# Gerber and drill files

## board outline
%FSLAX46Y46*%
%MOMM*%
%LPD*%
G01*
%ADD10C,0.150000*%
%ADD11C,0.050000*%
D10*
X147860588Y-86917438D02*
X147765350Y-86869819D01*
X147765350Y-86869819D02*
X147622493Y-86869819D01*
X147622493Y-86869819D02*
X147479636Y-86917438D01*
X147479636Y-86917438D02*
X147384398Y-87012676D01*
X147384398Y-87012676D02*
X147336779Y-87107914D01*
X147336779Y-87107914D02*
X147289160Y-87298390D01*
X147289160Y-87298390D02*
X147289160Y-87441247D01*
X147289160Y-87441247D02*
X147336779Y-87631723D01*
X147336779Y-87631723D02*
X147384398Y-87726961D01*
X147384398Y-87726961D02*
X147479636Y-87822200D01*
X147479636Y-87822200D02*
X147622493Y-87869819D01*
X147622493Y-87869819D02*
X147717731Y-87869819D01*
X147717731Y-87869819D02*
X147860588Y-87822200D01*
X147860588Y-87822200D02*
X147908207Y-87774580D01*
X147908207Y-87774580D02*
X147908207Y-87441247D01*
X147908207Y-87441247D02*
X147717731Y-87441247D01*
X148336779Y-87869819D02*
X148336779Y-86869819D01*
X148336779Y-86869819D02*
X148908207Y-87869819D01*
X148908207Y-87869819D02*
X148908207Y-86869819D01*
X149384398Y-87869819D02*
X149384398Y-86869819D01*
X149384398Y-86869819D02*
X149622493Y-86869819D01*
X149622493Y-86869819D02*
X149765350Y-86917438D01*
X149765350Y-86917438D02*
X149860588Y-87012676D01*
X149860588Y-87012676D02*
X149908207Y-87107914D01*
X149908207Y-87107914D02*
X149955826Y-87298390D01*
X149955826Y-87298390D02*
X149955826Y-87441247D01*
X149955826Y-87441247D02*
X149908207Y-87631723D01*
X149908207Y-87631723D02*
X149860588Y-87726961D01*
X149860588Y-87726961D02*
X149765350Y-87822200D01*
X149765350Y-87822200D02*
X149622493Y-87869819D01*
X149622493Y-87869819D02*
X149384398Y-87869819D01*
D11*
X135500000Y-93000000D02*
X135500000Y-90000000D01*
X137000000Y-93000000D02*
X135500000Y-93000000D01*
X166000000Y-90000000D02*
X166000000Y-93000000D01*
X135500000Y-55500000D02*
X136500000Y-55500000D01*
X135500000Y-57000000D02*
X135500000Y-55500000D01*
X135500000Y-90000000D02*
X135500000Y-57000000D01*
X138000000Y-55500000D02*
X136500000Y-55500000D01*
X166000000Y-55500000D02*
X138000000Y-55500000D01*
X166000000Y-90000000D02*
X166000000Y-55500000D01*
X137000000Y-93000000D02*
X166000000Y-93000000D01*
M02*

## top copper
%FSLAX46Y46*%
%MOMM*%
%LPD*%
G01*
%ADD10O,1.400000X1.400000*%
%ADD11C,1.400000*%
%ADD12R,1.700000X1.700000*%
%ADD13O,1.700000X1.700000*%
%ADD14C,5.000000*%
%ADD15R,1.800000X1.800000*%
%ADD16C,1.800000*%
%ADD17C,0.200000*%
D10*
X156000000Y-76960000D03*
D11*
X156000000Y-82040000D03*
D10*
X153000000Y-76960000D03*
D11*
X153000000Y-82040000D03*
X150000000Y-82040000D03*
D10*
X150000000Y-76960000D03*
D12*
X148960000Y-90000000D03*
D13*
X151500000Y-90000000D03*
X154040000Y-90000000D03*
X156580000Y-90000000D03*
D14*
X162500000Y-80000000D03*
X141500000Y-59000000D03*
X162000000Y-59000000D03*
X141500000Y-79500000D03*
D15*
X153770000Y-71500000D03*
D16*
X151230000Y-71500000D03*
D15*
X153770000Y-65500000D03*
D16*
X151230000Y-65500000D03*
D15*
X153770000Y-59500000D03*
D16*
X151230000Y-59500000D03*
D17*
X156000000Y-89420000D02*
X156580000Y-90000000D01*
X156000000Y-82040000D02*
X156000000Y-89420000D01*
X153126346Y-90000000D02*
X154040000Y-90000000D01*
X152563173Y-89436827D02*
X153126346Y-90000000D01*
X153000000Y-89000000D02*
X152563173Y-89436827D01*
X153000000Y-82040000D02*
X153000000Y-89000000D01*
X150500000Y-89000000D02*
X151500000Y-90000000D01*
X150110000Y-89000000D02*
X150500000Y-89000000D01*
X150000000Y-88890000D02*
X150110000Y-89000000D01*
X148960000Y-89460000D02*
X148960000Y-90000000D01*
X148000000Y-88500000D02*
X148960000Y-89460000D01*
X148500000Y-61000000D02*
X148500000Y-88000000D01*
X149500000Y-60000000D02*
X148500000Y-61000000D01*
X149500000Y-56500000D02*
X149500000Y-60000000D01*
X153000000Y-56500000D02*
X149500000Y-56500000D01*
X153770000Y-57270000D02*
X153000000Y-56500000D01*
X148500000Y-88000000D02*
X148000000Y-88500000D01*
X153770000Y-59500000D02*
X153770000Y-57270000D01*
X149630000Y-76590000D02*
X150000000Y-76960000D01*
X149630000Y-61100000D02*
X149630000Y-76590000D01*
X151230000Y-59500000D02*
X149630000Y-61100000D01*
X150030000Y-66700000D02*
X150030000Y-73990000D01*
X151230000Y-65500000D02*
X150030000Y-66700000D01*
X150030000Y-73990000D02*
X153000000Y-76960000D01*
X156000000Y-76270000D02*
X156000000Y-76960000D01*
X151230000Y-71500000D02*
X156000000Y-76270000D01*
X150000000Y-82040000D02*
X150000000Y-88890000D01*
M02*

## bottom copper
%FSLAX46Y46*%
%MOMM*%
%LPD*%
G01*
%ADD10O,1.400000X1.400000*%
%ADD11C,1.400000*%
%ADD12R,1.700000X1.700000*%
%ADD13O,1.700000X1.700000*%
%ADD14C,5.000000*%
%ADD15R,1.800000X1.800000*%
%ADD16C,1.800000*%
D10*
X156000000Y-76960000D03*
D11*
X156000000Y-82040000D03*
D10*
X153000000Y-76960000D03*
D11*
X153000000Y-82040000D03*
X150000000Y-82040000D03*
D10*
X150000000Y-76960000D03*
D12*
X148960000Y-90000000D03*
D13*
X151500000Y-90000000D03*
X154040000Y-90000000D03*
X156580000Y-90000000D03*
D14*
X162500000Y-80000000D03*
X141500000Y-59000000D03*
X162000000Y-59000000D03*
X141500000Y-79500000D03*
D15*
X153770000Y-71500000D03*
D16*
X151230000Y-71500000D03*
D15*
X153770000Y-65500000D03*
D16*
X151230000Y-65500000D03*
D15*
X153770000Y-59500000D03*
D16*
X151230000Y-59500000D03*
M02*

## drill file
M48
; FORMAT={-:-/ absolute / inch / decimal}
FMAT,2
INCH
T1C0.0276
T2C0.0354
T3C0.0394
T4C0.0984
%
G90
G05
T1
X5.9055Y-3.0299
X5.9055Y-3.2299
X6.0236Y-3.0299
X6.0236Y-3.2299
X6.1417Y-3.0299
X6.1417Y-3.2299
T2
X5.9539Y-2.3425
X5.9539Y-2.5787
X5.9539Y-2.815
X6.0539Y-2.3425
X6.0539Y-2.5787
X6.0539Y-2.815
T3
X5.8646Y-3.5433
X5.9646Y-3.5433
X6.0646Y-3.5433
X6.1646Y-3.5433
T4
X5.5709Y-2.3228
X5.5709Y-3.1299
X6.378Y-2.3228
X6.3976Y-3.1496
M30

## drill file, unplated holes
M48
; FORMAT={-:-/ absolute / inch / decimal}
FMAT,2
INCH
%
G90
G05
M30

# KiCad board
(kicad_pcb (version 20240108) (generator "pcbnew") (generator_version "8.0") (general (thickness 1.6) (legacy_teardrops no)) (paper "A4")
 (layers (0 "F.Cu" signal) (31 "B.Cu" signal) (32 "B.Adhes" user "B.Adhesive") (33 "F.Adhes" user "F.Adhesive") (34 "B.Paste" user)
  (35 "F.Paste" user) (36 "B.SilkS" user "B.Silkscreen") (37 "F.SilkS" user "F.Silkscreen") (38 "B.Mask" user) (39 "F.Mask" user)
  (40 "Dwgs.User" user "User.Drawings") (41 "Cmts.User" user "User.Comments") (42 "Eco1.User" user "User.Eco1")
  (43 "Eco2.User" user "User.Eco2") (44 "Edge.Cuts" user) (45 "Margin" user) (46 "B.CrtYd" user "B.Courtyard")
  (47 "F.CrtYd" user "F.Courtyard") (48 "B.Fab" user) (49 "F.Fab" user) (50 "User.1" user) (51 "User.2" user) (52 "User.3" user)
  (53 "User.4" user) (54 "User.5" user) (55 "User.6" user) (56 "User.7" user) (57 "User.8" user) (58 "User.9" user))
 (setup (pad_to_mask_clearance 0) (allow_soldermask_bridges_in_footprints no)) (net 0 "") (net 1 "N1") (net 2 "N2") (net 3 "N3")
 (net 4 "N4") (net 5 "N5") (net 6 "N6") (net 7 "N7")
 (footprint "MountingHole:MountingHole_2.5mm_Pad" (layer "F.Cu") (at 141.5 79.5)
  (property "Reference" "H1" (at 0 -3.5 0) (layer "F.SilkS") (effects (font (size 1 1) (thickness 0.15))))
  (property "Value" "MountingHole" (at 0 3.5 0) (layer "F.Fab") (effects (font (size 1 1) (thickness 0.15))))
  (pad "1" thru_hole circle (at 0 0) (size 5 5) (drill 2.5) (layers "*.Cu" "*.Mask") (remove_unused_layers no)))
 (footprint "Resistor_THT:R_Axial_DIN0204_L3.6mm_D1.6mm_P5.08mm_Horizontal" (layer "F.Cu") (at 156 82.04 90)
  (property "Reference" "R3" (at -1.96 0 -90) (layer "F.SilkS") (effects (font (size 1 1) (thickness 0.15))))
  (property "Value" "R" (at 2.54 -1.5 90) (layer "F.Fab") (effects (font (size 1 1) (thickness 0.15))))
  (pad "1" thru_hole circle (at 0 0 90) (size 1.4 1.4) (drill 0.7) (layers "*.Cu" "*.Mask") (remove_unused_layers no) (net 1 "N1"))
  (pad "2" thru_hole oval (at 5.08 0 90) (size 1.4 1.4) (drill 0.7) (layers "*.Cu" "*.Mask") (remove_unused_layers no) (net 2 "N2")))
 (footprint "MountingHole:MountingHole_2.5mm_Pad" (layer "F.Cu") (at 162.5 80)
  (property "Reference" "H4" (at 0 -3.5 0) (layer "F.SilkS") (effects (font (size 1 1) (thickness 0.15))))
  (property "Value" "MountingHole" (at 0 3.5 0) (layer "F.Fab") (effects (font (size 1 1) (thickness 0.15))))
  (pad "1" thru_hole circle (at 0 0) (size 5 5) (drill 2.5) (layers "*.Cu" "*.Mask") (remove_unused_layers no)))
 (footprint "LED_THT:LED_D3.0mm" (layer "F.Cu") (at 153.77 59.5 180)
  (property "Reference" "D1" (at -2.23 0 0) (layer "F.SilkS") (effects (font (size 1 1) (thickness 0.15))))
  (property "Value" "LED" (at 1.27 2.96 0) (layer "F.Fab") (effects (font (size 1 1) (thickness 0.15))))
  (pad "1" thru_hole rect (at 0 0 180) (size 1.8 1.8) (drill 0.9) (layers "*.Cu" "*.Mask") (remove_unused_layers no) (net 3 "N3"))
  (pad "2" thru_hole circle (at 2.54 0 180) (size 1.8 1.8) (drill 0.9) (layers "*.Cu" "*.Mask") (remove_unused_layers no) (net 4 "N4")))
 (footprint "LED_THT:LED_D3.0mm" (layer "F.Cu") (at 153.77 71.5 180)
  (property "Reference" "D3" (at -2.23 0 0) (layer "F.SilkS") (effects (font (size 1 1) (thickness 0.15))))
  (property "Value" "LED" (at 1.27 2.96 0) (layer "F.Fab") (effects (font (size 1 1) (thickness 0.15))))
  (pad "1" thru_hole rect (at 0 0 180) (size 1.8 1.8) (drill 0.9) (layers "*.Cu" "*.Mask") (remove_unused_layers no) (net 3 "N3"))
  (pad "2" thru_hole circle (at 2.54 0 180) (size 1.8 1.8) (drill 0.9) (layers "*.Cu" "*.Mask") (remove_unused_layers no) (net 2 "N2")))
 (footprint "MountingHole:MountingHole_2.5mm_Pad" (layer "F.Cu") (at 162 59)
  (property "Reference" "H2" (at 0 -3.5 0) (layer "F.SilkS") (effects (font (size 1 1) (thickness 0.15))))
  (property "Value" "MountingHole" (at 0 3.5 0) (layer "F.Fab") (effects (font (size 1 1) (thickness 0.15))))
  (pad "1" thru_hole circle (at 0 0) (size 5 5) (drill 2.5) (layers "*.Cu" "*.Mask") (remove_unused_layers no)))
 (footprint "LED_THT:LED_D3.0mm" (layer "F.Cu") (at 153.77 65.5 180)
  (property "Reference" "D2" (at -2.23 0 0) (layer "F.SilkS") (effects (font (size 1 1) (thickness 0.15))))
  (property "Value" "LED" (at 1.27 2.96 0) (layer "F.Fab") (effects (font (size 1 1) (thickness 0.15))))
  (pad "1" thru_hole rect (at 0 0 180) (size 1.8 1.8) (drill 0.9) (layers "*.Cu" "*.Mask") (remove_unused_layers no) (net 3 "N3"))
  (pad "2" thru_hole circle (at 2.54 0 180) (size 1.8 1.8) (drill 0.9) (layers "*.Cu" "*.Mask") (remove_unused_layers no) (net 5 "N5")))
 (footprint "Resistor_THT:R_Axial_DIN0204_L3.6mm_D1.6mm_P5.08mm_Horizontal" (layer "F.Cu") (at 153 82.04 90)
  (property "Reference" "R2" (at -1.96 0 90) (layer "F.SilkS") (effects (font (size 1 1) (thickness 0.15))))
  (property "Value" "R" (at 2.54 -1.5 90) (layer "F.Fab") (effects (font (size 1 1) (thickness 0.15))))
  (pad "1" thru_hole circle (at 0 0 90) (size 1.4 1.4) (drill 0.7) (layers "*.Cu" "*.Mask") (remove_unused_layers no) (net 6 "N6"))
  (pad "2" thru_hole oval (at 5.08 0 90) (size 1.4 1.4) (drill 0.7) (layers "*.Cu" "*.Mask") (remove_unused_layers no) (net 5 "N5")))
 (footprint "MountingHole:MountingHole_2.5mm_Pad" (layer "F.Cu") (at 141.5 59)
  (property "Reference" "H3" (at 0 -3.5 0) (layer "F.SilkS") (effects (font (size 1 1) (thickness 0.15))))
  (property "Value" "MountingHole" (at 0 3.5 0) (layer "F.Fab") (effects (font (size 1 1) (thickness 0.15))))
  (pad "1" thru_hole circle (at 0 0) (size 5 5) (drill 2.5) (layers "*.Cu" "*.Mask") (remove_unused_layers no)))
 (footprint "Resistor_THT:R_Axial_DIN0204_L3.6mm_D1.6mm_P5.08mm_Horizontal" (layer "F.Cu") (at 150 82.04 90)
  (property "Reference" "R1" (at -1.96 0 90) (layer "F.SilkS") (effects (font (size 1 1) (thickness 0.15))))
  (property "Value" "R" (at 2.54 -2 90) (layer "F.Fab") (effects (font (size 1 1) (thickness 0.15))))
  (pad "1" thru_hole circle (at 0 0 90) (size 1.4 1.4) (drill 0.7) (layers "*.Cu" "*.Mask") (remove_unused_layers no) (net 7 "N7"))
  (pad "2" thru_hole oval (at 5.08 0 90) (size 1.4 1.4) (drill 0.7) (layers "*.Cu" "*.Mask") (remove_unused_layers no) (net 4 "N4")))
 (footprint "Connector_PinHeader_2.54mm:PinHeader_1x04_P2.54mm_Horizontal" (layer "B.Cu") (at 148.96 90 -90)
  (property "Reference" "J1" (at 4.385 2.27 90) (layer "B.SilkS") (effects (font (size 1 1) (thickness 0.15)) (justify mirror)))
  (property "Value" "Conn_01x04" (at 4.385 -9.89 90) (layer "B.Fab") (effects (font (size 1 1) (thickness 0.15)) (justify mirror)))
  (pad "1" thru_hole rect (at 0 0 270) (size 1.7 1.7) (drill 1) (layers "*.Cu" "*.Mask") (remove_unused_layers no) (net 3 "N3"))
  (pad "2" thru_hole oval (at 0 -2.54 270) (size 1.7 1.7) (drill 1) (layers "*.Cu" "*.Mask") (remove_unused_layers no) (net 7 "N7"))
  (pad "3" thru_hole oval (at 0 -5.08 270) (size 1.7 1.7) (drill 1) (layers "*.Cu" "*.Mask") (remove_unused_layers no) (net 6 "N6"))
  (pad "4" thru_hole oval (at 0 -7.62 270) (size 1.7 1.7) (drill 1) (layers "*.Cu" "*.Mask") (remove_unused_layers no) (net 1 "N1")))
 (gr_line (start 166 55.5) (end 138 55.5) (stroke (width 0.05) (type default)) (layer "Edge.Cuts"))
 (gr_line (start 135.5 57) (end 135.5 55.5) (stroke (width 0.05) (type default)) (layer "Edge.Cuts"))
 (gr_line (start 137 93) (end 135.5 93) (stroke (width 0.05) (type default)) (layer "Edge.Cuts"))
 (gr_line (start 137 93) (end 166 93) (stroke (width 0.05) (type default)) (layer "Edge.Cuts"))
 (gr_line (start 138 55.5) (end 136.5 55.5) (stroke (width 0.05) (type default)) (layer "Edge.Cuts"))
 (gr_line (start 166 90) (end 166 93) (stroke (width 0.05) (type default)) (layer "Edge.Cuts"))
 (gr_line (start 135.5 93) (end 135.5 90) (stroke (width 0.05) (type default)) (layer "Edge.Cuts"))
 (gr_line (start 135.5 55.5) (end 136.5 55.5) (stroke (width 0.05) (type default)) (layer "Edge.Cuts"))
 (gr_line (start 166 90) (end 166 55.5) (stroke (width 0.05) (type default)) (layer "Edge.Cuts"))
 (gr_line (start 135.5 90) (end 135.5 57) (stroke (width 0.05) (type default)) (layer "Edge.Cuts"))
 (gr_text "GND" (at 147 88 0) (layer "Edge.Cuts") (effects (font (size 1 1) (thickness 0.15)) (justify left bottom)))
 (segment (start 149.5 56.5) (end 149.5 60) (width 0.2) (layer "F.Cu") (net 3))
 (segment (start 148.96 89.46) (end 148.96 90) (width 0.2) (layer "F.Cu") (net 3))
 (segment (start 153.77 59.5) (end 153.77 57.27) (width 0.2) (layer "F.Cu") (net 3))
 (segment (start 148.5 88) (end 148 88.5) (width 0.2) (layer "F.Cu") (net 3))
 (segment (start 149.5 60) (end 148.5 61) (width 0.2) (layer "F.Cu") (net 3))
 (segment (start 153 56.5) (end 149.5 56.5) (width 0.2) (layer "F.Cu") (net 3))
 (segment (start 148 88.5) (end 148.96 89.46) (width 0.2) (layer "F.Cu") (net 3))
 (segment (start 148.5 61) (end 148.5 88) (width 0.2) (layer "F.Cu") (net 3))
 (segment (start 153.77 57.27) (end 153 56.5) (width 0.2) (layer "F.Cu") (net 3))
 (segment (start 149.63 76.59) (end 150 76.96) (width 0.2) (layer "F.Cu") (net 4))
 (segment (start 149.63 61.1) (end 149.63 76.59) (width 0.2) (layer "F.Cu") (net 4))
 (segment (start 151.23 59.5) (end 149.63 61.1) (width 0.2) (layer "F.Cu") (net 4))
 (segment (start 150.03 66.7) (end 150.03 73.99) (width 0.2) (layer "F.Cu") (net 5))
 (segment (start 150.03 73.99) (end 153 76.96) (width 0.2) (layer "F.Cu") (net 5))
 (segment (start 151.23 65.5) (end 150.03 66.7) (width 0.2) (layer "F.Cu") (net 5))
 (segment (start 156 76.27) (end 156 76.96) (width 0.2) (layer "F.Cu") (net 2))
 (segment (start 151.23 71.5) (end 156 76.27) (width 0.2) (layer "F.Cu") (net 2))
 (segment (start 153 82.04) (end 153 89) (width 0.2) (layer "F.Cu") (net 6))
 (segment (start 152.563173 89.436827) (end 153.126346 90) (width 0.2) (layer "F.Cu") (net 6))
 (segment (start 153.126346 90) (end 154.04 90) (width 0.2) (layer "F.Cu") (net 6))
 (segment (start 153 89) (end 152.563173 89.436827) (width 0.2) (layer "F.Cu") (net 6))
 (segment (start 156 89.42) (end 156.58 90) (width 0.2) (layer "F.Cu") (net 1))
 (segment (start 156 82.04) (end 156 89.42) (width 0.2) (layer "F.Cu") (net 1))
 (segment (start 150 82.04) (end 150 88.89) (width 0.2) (layer "F.Cu") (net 7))
 (segment (start 150.5 89) (end 151.5 90) (width 0.2) (layer "F.Cu") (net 7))
 (segment (start 150.11 89) (end 150.5 89) (width 0.2) (layer "F.Cu") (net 7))
 (segment (start 150 88.89) (end 150.11 89) (width 0.2) (layer "F.Cu") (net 7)))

